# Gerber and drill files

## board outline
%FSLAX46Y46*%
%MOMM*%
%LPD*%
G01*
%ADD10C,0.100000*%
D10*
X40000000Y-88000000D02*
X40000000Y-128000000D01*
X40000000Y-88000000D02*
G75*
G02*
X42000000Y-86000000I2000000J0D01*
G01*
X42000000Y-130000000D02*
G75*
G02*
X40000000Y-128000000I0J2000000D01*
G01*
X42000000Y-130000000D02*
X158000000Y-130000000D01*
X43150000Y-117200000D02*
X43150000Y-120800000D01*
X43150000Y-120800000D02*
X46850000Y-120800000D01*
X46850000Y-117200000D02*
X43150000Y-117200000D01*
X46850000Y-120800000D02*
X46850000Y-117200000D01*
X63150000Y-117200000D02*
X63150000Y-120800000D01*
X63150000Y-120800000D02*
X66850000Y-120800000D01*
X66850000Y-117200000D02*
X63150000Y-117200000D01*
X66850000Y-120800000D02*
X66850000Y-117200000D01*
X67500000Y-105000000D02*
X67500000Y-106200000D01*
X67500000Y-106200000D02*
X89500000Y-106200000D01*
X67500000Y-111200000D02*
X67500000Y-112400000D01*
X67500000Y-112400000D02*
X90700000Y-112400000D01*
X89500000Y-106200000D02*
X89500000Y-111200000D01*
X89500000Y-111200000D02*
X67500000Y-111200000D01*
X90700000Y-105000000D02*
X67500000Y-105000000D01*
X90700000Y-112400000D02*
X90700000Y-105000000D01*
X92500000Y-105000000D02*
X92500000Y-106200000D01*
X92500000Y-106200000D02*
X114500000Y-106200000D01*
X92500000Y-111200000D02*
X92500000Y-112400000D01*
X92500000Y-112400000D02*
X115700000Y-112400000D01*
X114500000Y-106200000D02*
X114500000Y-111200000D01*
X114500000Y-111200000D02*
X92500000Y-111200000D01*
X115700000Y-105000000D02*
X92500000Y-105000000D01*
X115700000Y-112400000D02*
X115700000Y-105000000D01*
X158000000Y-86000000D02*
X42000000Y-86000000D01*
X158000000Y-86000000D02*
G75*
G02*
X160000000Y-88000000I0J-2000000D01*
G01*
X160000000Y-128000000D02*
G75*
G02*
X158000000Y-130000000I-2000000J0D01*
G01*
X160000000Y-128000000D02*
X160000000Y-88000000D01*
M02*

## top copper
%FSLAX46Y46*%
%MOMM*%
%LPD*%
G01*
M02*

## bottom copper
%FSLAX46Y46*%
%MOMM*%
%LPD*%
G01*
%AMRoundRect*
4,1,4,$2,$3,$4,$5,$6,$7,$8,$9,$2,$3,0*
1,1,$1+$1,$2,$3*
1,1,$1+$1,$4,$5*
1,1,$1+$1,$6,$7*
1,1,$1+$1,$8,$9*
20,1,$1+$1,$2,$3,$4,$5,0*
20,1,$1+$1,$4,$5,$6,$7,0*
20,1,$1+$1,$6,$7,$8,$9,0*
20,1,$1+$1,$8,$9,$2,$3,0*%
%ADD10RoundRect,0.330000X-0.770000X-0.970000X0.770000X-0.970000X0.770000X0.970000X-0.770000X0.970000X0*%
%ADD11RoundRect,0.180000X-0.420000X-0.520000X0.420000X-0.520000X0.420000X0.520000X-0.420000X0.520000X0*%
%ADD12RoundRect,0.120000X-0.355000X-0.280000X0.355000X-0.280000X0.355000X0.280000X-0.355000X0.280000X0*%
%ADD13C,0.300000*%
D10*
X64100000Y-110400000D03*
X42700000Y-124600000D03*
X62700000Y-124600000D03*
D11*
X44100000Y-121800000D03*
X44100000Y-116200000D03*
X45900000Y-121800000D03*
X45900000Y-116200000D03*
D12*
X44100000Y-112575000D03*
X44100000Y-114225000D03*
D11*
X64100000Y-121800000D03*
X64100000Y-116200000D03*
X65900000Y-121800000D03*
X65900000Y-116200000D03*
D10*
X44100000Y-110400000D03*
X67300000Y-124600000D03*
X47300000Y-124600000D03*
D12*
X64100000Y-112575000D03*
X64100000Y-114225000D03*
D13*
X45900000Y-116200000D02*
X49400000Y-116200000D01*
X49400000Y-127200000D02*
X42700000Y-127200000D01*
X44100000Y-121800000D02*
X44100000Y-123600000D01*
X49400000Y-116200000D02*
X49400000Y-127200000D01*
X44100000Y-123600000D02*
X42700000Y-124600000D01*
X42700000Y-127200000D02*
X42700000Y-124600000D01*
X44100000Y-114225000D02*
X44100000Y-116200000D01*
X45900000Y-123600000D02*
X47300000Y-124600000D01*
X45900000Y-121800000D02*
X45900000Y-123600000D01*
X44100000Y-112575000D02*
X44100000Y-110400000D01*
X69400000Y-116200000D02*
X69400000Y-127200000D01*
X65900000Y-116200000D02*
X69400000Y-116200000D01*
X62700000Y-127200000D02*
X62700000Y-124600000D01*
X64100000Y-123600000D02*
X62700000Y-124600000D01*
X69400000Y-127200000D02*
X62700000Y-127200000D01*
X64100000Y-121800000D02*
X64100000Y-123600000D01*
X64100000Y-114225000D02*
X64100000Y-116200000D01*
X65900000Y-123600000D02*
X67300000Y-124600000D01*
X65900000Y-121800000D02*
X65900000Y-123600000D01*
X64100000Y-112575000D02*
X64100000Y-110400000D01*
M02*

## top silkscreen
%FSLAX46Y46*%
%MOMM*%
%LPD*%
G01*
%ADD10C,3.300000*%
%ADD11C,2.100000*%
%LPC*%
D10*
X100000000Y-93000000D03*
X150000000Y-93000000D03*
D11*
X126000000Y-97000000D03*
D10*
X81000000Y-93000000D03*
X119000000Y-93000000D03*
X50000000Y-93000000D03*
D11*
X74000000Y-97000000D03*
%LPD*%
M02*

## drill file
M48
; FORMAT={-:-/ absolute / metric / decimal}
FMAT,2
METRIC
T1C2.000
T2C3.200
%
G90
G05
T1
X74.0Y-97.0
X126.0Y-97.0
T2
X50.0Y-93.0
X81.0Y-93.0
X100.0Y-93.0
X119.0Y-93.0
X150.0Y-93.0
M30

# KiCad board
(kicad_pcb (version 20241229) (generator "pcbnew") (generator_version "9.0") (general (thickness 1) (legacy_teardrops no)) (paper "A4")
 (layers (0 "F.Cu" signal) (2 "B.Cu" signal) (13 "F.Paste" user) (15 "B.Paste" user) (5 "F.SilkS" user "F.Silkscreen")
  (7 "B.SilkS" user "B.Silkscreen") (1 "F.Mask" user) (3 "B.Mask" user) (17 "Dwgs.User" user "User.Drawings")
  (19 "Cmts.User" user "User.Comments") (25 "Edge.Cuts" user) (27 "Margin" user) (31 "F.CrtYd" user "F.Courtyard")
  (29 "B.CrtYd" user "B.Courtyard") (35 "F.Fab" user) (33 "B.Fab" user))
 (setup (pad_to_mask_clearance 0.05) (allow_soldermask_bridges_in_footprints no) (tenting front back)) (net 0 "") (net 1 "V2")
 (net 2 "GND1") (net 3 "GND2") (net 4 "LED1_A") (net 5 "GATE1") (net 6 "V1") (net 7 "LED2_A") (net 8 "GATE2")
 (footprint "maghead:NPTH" (layer "F.Cu") (at 100 93)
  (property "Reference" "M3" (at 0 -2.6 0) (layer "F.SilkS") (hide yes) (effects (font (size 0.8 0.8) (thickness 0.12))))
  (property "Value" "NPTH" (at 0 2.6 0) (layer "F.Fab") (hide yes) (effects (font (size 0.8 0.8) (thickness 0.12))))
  (pad "" np_thru_hole circle (at 0 0) (size 3.2 3.2) (drill 3.2) (layers "*.Cu" "*.Mask")))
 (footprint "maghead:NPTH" (layer "F.Cu") (at 150 93)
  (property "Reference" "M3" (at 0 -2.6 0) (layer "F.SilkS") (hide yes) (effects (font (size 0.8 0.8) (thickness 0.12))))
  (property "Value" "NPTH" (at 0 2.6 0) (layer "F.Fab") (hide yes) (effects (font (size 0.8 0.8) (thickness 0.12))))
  (pad "" np_thru_hole circle (at 0 0) (size 3.2 3.2) (drill 3.2) (layers "*.Cu" "*.Mask")))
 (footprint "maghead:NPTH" (layer "F.Cu") (at 126 97)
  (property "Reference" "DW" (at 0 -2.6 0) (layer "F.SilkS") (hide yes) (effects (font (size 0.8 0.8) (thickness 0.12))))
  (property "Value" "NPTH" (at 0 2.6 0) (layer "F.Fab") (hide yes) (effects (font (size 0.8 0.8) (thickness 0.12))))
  (pad "" np_thru_hole circle (at 0 0) (size 2 2) (drill 2) (layers "*.Cu" "*.Mask")))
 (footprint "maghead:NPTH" (layer "F.Cu") (at 81 93)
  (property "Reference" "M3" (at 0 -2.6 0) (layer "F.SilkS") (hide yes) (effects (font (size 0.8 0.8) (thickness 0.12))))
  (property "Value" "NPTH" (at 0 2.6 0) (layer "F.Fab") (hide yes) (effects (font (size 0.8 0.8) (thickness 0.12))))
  (pad "" np_thru_hole circle (at 0 0) (size 3.2 3.2) (drill 3.2) (layers "*.Cu" "*.Mask")))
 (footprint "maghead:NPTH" (layer "F.Cu") (at 119 93)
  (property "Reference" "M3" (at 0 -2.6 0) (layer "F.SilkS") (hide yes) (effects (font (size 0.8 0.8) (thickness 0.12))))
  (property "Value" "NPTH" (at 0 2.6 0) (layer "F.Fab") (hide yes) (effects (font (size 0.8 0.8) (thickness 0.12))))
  (pad "" np_thru_hole circle (at 0 0) (size 3.2 3.2) (drill 3.2) (layers "*.Cu" "*.Mask")))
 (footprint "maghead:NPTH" (layer "F.Cu") (at 50 93)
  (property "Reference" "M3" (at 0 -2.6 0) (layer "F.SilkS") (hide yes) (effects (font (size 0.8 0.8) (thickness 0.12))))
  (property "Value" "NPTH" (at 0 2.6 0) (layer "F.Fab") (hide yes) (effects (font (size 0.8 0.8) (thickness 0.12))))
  (pad "" np_thru_hole circle (at 0 0) (size 3.2 3.2) (drill 3.2) (layers "*.Cu" "*.Mask")))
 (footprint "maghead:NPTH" (layer "F.Cu") (at 74 97)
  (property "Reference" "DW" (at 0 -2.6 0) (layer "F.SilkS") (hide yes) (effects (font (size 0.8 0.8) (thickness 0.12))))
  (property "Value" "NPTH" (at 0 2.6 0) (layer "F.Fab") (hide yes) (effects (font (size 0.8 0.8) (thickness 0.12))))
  (pad "" np_thru_hole circle (at 0 0) (size 2 2) (drill 2) (layers "*.Cu" "*.Mask")))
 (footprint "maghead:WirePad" (layer "B.Cu") (at 64.1 110.4)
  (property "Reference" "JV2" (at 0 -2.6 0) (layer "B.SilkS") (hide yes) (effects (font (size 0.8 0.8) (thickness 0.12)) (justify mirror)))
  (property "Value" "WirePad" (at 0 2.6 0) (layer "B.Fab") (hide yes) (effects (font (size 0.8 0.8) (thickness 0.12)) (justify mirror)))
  (pad "1" smd roundrect (at 0 0) (size 2.2 2.6) (layers "B.Cu" "B.Mask") (roundrect_rratio 0.15) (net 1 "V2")))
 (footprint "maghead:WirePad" (layer "B.Cu") (at 42.7 124.6)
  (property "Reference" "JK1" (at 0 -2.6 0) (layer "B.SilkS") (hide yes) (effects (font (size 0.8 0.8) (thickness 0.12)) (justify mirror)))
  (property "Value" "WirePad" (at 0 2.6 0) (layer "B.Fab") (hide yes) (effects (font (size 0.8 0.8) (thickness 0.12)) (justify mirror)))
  (pad "1" smd roundrect (at 0 0) (size 2.2 2.6) (layers "B.Cu" "B.Mask") (roundrect_rratio 0.15) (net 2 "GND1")))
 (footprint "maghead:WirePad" (layer "B.Cu") (at 62.7 124.6)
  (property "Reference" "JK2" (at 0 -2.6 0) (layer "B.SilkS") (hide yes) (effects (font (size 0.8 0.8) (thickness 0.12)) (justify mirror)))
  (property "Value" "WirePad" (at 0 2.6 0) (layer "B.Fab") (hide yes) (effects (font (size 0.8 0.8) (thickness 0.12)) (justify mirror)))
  (pad "1" smd roundrect (at 0 0) (size 2.2 2.6) (layers "B.Cu" "B.Mask") (roundrect_rratio 0.15) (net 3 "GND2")))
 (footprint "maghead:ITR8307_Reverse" (layer "B.Cu") (at 45 119)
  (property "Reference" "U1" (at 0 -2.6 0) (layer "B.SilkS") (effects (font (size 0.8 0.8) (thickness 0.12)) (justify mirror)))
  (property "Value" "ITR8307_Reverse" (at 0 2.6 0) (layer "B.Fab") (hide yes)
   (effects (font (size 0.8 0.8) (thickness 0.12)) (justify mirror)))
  (pad "1" smd roundrect (at -0.9 2.8) (size 1.2 1.4) (layers "B.Cu" "B.Mask" "B.Paste") (roundrect_rratio 0.15) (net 2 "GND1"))
  (pad "2" smd roundrect (at -0.9 -2.8) (size 1.2 1.4) (layers "B.Cu" "B.Mask" "B.Paste") (roundrect_rratio 0.15) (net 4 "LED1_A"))
  (pad "3" smd roundrect (at 0.9 2.8) (size 1.2 1.4) (layers "B.Cu" "B.Mask" "B.Paste") (roundrect_rratio 0.15) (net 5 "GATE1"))
  (pad "4" smd roundrect (at 0.9 -2.8) (size 1.2 1.4) (layers "B.Cu" "B.Mask" "B.Paste") (roundrect_rratio 0.15) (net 2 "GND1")))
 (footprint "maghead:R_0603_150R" (layer "B.Cu") (at 44.1 113.4)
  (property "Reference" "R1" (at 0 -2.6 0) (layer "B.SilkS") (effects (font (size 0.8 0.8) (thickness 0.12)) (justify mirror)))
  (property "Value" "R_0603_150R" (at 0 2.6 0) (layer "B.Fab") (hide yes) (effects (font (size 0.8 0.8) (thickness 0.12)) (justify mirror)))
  (pad "1" smd roundrect (at 0 -0.825) (size 0.95 0.8) (layers "B.Cu" "B.Mask" "B.Paste") (roundrect_rratio 0.15) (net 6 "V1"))
  (pad "2" smd roundrect (at 0 0.825) (size 0.95 0.8) (layers "B.Cu" "B.Mask" "B.Paste") (roundrect_rratio 0.15) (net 4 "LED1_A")))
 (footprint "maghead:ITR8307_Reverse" (layer "B.Cu") (at 65 119)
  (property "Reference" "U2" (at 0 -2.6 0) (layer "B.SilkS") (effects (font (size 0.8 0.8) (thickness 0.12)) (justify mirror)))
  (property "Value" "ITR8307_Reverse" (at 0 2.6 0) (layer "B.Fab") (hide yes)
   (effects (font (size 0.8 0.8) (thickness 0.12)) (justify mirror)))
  (pad "1" smd roundrect (at -0.9 2.8) (size 1.2 1.4) (layers "B.Cu" "B.Mask" "B.Paste") (roundrect_rratio 0.15) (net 3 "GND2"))
  (pad "2" smd roundrect (at -0.9 -2.8) (size 1.2 1.4) (layers "B.Cu" "B.Mask" "B.Paste") (roundrect_rratio 0.15) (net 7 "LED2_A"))
  (pad "3" smd roundrect (at 0.9 2.8) (size 1.2 1.4) (layers "B.Cu" "B.Mask" "B.Paste") (roundrect_rratio 0.15) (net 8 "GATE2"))
  (pad "4" smd roundrect (at 0.9 -2.8) (size 1.2 1.4) (layers "B.Cu" "B.Mask" "B.Paste") (roundrect_rratio 0.15) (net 3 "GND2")))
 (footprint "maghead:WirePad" (layer "B.Cu") (at 44.1 110.4)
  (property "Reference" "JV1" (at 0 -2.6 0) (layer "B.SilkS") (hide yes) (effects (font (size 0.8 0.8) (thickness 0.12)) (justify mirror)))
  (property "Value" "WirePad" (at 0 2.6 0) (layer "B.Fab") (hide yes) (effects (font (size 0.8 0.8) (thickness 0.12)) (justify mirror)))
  (pad "1" smd roundrect (at 0 0) (size 2.2 2.6) (layers "B.Cu" "B.Mask") (roundrect_rratio 0.15) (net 6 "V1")))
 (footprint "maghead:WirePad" (layer "B.Cu") (at 67.3 124.6)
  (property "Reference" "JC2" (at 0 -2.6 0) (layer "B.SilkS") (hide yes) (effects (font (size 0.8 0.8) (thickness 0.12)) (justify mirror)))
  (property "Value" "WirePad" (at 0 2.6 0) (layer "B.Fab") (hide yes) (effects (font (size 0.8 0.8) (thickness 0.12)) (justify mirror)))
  (pad "1" smd roundrect (at 0 0) (size 2.2 2.6) (layers "B.Cu" "B.Mask") (roundrect_rratio 0.15) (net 8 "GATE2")))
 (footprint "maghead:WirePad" (layer "B.Cu") (at 47.3 124.6)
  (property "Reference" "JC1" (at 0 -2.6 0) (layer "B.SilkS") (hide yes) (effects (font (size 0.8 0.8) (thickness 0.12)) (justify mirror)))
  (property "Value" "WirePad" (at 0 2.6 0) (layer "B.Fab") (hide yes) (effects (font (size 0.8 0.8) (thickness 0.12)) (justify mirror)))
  (pad "1" smd roundrect (at 0 0) (size 2.2 2.6) (layers "B.Cu" "B.Mask") (roundrect_rratio 0.15) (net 5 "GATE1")))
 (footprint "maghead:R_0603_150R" (layer "B.Cu") (at 64.1 113.4)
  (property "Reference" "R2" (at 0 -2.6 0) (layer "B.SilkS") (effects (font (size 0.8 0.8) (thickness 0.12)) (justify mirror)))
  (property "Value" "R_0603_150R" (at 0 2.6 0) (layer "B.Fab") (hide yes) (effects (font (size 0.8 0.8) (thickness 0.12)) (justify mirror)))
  (pad "1" smd roundrect (at 0 -0.825) (size 0.95 0.8) (layers "B.Cu" "B.Mask" "B.Paste") (roundrect_rratio 0.15) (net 1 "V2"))
  (pad "2" smd roundrect (at 0 0.825) (size 0.95 0.8) (layers "B.Cu" "B.Mask" "B.Paste") (roundrect_rratio 0.15) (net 7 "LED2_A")))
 (gr_line (start 40 88) (end 40 128) (stroke (width 0.1) (type solid)) (layer "Edge.Cuts"))
 (gr_arc (start 40 88) (mid 40.585786 86.585786) (end 42 86) (stroke (width 0.1) (type solid)) (layer "Edge.Cuts"))
 (gr_arc (start 42 130) (mid 40.585801 129.414199) (end 40 128) (stroke (width 0.1) (type solid)) (layer "Edge.Cuts"))
 (gr_line (start 42 130) (end 158 130) (stroke (width 0.1) (type solid)) (layer "Edge.Cuts"))
 (gr_line (start 43.15 117.2) (end 43.15 120.8) (stroke (width 0.1) (type solid)) (layer "Edge.Cuts"))
 (gr_line (start 43.15 120.8) (end 46.85 120.8) (stroke (width 0.1) (type solid)) (layer "Edge.Cuts"))
 (gr_line (start 46.85 117.2) (end 43.15 117.2) (stroke (width 0.1) (type solid)) (layer "Edge.Cuts"))
 (gr_line (start 46.85 120.8) (end 46.85 117.2) (stroke (width 0.1) (type solid)) (layer "Edge.Cuts"))
 (gr_line (start 63.15 117.2) (end 63.15 120.8) (stroke (width 0.1) (type solid)) (layer "Edge.Cuts"))
 (gr_line (start 63.15 120.8) (end 66.85 120.8) (stroke (width 0.1) (type solid)) (layer "Edge.Cuts"))
 (gr_line (start 66.85 117.2) (end 63.15 117.2) (stroke (width 0.1) (type solid)) (layer "Edge.Cuts"))
 (gr_line (start 66.85 120.8) (end 66.85 117.2) (stroke (width 0.1) (type solid)) (layer "Edge.Cuts"))
 (gr_line (start 67.5 105) (end 67.5 106.2) (stroke (width 0.1) (type solid)) (layer "Edge.Cuts"))
 (gr_line (start 67.5 106.2) (end 89.5 106.2) (stroke (width 0.1) (type solid)) (layer "Edge.Cuts"))
 (gr_line (start 67.5 111.2) (end 67.5 112.4) (stroke (width 0.1) (type solid)) (layer "Edge.Cuts"))
 (gr_line (start 67.5 112.4) (end 90.7 112.4) (stroke (width 0.1) (type solid)) (layer "Edge.Cuts"))
 (gr_line (start 89.5 106.2) (end 89.5 111.2) (stroke (width 0.1) (type solid)) (layer "Edge.Cuts"))
 (gr_line (start 89.5 111.2) (end 67.5 111.2) (stroke (width 0.1) (type solid)) (layer "Edge.Cuts"))
 (gr_line (start 90.7 105) (end 67.5 105) (stroke (width 0.1) (type solid)) (layer "Edge.Cuts"))
 (gr_line (start 90.7 112.4) (end 90.7 105) (stroke (width 0.1) (type solid)) (layer "Edge.Cuts"))
 (gr_line (start 92.5 105) (end 92.5 106.2) (stroke (width 0.1) (type solid)) (layer "Edge.Cuts"))
 (gr_line (start 92.5 106.2) (end 114.5 106.2) (stroke (width 0.1) (type solid)) (layer "Edge.Cuts"))
 (gr_line (start 92.5 111.2) (end 92.5 112.4) (stroke (width 0.1) (type solid)) (layer "Edge.Cuts"))
 (gr_line (start 92.5 112.4) (end 115.7 112.4) (stroke (width 0.1) (type solid)) (layer "Edge.Cuts"))
 (gr_line (start 114.5 106.2) (end 114.5 111.2) (stroke (width 0.1) (type solid)) (layer "Edge.Cuts"))
 (gr_line (start 114.5 111.2) (end 92.5 111.2) (stroke (width 0.1) (type solid)) (layer "Edge.Cuts"))
 (gr_line (start 115.7 105) (end 92.5 105) (stroke (width 0.1) (type solid)) (layer "Edge.Cuts"))
 (gr_line (start 115.7 112.4) (end 115.7 105) (stroke (width 0.1) (type solid)) (layer "Edge.Cuts"))
 (gr_line (start 158 86) (end 42 86) (stroke (width 0.1) (type solid)) (layer "Edge.Cuts"))
 (gr_arc (start 158 86) (mid 159.414214 86.585786) (end 160 88) (stroke (width 0.1) (type solid)) (layer "Edge.Cuts"))
 (gr_arc (start 160 128) (mid 159.414214 129.414214) (end 158 130) (stroke (width 0.1) (type solid)) (layer "Edge.Cuts"))
 (gr_line (start 160 128) (end 160 88) (stroke (width 0.1) (type solid)) (layer "Edge.Cuts"))
 (segment (start 45.9 116.2) (end 49.4 116.2) (width 0.3) (layer "B.Cu") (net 2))
 (segment (start 49.4 127.2) (end 42.7 127.2) (width 0.3) (layer "B.Cu") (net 2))
 (segment (start 44.1 121.8) (end 44.1 123.6) (width 0.3) (layer "B.Cu") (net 2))
 (segment (start 49.4 116.2) (end 49.4 127.2) (width 0.3) (layer "B.Cu") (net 2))
 (segment (start 44.1 123.6) (end 42.7 124.6) (width 0.3) (layer "B.Cu") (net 2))
 (segment (start 42.7 127.2) (end 42.7 124.6) (width 0.3) (layer "B.Cu") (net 2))
 (segment (start 44.1 114.225) (end 44.1 116.2) (width 0.3) (layer "B.Cu") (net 4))
 (segment (start 45.9 123.6) (end 47.3 124.6) (width 0.3) (layer "B.Cu") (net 5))
 (segment (start 45.9 121.8) (end 45.9 123.6) (width 0.3) (layer "B.Cu") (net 5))
 (segment (start 44.1 112.575) (end 44.1 110.4) (width 0.3) (layer "B.Cu") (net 6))
 (segment (start 69.4 116.2) (end 69.4 127.2) (width 0.3) (layer "B.Cu") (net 3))
 (segment (start 65.9 116.2) (end 69.4 116.2) (width 0.3) (layer "B.Cu") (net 3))
 (segment (start 62.7 127.2) (end 62.7 124.6) (width 0.3) (layer "B.Cu") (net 3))
 (segment (start 64.1 123.6) (end 62.7 124.6) (width 0.3) (layer "B.Cu") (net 3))
 (segment (start 69.4 127.2) (end 62.7 127.2) (width 0.3) (layer "B.Cu") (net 3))
 (segment (start 64.1 121.8) (end 64.1 123.6) (width 0.3) (layer "B.Cu") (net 3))
 (segment (start 64.1 114.225) (end 64.1 116.2) (width 0.3) (layer "B.Cu") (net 7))
 (segment (start 65.9 123.6) (end 67.3 124.6) (width 0.3) (layer "B.Cu") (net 8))
 (segment (start 65.9 121.8) (end 65.9 123.6) (width 0.3) (layer "B.Cu") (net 8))
 (segment (start 64.1 112.575) (end 64.1 110.4) (width 0.3) (layer "B.Cu") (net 1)))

